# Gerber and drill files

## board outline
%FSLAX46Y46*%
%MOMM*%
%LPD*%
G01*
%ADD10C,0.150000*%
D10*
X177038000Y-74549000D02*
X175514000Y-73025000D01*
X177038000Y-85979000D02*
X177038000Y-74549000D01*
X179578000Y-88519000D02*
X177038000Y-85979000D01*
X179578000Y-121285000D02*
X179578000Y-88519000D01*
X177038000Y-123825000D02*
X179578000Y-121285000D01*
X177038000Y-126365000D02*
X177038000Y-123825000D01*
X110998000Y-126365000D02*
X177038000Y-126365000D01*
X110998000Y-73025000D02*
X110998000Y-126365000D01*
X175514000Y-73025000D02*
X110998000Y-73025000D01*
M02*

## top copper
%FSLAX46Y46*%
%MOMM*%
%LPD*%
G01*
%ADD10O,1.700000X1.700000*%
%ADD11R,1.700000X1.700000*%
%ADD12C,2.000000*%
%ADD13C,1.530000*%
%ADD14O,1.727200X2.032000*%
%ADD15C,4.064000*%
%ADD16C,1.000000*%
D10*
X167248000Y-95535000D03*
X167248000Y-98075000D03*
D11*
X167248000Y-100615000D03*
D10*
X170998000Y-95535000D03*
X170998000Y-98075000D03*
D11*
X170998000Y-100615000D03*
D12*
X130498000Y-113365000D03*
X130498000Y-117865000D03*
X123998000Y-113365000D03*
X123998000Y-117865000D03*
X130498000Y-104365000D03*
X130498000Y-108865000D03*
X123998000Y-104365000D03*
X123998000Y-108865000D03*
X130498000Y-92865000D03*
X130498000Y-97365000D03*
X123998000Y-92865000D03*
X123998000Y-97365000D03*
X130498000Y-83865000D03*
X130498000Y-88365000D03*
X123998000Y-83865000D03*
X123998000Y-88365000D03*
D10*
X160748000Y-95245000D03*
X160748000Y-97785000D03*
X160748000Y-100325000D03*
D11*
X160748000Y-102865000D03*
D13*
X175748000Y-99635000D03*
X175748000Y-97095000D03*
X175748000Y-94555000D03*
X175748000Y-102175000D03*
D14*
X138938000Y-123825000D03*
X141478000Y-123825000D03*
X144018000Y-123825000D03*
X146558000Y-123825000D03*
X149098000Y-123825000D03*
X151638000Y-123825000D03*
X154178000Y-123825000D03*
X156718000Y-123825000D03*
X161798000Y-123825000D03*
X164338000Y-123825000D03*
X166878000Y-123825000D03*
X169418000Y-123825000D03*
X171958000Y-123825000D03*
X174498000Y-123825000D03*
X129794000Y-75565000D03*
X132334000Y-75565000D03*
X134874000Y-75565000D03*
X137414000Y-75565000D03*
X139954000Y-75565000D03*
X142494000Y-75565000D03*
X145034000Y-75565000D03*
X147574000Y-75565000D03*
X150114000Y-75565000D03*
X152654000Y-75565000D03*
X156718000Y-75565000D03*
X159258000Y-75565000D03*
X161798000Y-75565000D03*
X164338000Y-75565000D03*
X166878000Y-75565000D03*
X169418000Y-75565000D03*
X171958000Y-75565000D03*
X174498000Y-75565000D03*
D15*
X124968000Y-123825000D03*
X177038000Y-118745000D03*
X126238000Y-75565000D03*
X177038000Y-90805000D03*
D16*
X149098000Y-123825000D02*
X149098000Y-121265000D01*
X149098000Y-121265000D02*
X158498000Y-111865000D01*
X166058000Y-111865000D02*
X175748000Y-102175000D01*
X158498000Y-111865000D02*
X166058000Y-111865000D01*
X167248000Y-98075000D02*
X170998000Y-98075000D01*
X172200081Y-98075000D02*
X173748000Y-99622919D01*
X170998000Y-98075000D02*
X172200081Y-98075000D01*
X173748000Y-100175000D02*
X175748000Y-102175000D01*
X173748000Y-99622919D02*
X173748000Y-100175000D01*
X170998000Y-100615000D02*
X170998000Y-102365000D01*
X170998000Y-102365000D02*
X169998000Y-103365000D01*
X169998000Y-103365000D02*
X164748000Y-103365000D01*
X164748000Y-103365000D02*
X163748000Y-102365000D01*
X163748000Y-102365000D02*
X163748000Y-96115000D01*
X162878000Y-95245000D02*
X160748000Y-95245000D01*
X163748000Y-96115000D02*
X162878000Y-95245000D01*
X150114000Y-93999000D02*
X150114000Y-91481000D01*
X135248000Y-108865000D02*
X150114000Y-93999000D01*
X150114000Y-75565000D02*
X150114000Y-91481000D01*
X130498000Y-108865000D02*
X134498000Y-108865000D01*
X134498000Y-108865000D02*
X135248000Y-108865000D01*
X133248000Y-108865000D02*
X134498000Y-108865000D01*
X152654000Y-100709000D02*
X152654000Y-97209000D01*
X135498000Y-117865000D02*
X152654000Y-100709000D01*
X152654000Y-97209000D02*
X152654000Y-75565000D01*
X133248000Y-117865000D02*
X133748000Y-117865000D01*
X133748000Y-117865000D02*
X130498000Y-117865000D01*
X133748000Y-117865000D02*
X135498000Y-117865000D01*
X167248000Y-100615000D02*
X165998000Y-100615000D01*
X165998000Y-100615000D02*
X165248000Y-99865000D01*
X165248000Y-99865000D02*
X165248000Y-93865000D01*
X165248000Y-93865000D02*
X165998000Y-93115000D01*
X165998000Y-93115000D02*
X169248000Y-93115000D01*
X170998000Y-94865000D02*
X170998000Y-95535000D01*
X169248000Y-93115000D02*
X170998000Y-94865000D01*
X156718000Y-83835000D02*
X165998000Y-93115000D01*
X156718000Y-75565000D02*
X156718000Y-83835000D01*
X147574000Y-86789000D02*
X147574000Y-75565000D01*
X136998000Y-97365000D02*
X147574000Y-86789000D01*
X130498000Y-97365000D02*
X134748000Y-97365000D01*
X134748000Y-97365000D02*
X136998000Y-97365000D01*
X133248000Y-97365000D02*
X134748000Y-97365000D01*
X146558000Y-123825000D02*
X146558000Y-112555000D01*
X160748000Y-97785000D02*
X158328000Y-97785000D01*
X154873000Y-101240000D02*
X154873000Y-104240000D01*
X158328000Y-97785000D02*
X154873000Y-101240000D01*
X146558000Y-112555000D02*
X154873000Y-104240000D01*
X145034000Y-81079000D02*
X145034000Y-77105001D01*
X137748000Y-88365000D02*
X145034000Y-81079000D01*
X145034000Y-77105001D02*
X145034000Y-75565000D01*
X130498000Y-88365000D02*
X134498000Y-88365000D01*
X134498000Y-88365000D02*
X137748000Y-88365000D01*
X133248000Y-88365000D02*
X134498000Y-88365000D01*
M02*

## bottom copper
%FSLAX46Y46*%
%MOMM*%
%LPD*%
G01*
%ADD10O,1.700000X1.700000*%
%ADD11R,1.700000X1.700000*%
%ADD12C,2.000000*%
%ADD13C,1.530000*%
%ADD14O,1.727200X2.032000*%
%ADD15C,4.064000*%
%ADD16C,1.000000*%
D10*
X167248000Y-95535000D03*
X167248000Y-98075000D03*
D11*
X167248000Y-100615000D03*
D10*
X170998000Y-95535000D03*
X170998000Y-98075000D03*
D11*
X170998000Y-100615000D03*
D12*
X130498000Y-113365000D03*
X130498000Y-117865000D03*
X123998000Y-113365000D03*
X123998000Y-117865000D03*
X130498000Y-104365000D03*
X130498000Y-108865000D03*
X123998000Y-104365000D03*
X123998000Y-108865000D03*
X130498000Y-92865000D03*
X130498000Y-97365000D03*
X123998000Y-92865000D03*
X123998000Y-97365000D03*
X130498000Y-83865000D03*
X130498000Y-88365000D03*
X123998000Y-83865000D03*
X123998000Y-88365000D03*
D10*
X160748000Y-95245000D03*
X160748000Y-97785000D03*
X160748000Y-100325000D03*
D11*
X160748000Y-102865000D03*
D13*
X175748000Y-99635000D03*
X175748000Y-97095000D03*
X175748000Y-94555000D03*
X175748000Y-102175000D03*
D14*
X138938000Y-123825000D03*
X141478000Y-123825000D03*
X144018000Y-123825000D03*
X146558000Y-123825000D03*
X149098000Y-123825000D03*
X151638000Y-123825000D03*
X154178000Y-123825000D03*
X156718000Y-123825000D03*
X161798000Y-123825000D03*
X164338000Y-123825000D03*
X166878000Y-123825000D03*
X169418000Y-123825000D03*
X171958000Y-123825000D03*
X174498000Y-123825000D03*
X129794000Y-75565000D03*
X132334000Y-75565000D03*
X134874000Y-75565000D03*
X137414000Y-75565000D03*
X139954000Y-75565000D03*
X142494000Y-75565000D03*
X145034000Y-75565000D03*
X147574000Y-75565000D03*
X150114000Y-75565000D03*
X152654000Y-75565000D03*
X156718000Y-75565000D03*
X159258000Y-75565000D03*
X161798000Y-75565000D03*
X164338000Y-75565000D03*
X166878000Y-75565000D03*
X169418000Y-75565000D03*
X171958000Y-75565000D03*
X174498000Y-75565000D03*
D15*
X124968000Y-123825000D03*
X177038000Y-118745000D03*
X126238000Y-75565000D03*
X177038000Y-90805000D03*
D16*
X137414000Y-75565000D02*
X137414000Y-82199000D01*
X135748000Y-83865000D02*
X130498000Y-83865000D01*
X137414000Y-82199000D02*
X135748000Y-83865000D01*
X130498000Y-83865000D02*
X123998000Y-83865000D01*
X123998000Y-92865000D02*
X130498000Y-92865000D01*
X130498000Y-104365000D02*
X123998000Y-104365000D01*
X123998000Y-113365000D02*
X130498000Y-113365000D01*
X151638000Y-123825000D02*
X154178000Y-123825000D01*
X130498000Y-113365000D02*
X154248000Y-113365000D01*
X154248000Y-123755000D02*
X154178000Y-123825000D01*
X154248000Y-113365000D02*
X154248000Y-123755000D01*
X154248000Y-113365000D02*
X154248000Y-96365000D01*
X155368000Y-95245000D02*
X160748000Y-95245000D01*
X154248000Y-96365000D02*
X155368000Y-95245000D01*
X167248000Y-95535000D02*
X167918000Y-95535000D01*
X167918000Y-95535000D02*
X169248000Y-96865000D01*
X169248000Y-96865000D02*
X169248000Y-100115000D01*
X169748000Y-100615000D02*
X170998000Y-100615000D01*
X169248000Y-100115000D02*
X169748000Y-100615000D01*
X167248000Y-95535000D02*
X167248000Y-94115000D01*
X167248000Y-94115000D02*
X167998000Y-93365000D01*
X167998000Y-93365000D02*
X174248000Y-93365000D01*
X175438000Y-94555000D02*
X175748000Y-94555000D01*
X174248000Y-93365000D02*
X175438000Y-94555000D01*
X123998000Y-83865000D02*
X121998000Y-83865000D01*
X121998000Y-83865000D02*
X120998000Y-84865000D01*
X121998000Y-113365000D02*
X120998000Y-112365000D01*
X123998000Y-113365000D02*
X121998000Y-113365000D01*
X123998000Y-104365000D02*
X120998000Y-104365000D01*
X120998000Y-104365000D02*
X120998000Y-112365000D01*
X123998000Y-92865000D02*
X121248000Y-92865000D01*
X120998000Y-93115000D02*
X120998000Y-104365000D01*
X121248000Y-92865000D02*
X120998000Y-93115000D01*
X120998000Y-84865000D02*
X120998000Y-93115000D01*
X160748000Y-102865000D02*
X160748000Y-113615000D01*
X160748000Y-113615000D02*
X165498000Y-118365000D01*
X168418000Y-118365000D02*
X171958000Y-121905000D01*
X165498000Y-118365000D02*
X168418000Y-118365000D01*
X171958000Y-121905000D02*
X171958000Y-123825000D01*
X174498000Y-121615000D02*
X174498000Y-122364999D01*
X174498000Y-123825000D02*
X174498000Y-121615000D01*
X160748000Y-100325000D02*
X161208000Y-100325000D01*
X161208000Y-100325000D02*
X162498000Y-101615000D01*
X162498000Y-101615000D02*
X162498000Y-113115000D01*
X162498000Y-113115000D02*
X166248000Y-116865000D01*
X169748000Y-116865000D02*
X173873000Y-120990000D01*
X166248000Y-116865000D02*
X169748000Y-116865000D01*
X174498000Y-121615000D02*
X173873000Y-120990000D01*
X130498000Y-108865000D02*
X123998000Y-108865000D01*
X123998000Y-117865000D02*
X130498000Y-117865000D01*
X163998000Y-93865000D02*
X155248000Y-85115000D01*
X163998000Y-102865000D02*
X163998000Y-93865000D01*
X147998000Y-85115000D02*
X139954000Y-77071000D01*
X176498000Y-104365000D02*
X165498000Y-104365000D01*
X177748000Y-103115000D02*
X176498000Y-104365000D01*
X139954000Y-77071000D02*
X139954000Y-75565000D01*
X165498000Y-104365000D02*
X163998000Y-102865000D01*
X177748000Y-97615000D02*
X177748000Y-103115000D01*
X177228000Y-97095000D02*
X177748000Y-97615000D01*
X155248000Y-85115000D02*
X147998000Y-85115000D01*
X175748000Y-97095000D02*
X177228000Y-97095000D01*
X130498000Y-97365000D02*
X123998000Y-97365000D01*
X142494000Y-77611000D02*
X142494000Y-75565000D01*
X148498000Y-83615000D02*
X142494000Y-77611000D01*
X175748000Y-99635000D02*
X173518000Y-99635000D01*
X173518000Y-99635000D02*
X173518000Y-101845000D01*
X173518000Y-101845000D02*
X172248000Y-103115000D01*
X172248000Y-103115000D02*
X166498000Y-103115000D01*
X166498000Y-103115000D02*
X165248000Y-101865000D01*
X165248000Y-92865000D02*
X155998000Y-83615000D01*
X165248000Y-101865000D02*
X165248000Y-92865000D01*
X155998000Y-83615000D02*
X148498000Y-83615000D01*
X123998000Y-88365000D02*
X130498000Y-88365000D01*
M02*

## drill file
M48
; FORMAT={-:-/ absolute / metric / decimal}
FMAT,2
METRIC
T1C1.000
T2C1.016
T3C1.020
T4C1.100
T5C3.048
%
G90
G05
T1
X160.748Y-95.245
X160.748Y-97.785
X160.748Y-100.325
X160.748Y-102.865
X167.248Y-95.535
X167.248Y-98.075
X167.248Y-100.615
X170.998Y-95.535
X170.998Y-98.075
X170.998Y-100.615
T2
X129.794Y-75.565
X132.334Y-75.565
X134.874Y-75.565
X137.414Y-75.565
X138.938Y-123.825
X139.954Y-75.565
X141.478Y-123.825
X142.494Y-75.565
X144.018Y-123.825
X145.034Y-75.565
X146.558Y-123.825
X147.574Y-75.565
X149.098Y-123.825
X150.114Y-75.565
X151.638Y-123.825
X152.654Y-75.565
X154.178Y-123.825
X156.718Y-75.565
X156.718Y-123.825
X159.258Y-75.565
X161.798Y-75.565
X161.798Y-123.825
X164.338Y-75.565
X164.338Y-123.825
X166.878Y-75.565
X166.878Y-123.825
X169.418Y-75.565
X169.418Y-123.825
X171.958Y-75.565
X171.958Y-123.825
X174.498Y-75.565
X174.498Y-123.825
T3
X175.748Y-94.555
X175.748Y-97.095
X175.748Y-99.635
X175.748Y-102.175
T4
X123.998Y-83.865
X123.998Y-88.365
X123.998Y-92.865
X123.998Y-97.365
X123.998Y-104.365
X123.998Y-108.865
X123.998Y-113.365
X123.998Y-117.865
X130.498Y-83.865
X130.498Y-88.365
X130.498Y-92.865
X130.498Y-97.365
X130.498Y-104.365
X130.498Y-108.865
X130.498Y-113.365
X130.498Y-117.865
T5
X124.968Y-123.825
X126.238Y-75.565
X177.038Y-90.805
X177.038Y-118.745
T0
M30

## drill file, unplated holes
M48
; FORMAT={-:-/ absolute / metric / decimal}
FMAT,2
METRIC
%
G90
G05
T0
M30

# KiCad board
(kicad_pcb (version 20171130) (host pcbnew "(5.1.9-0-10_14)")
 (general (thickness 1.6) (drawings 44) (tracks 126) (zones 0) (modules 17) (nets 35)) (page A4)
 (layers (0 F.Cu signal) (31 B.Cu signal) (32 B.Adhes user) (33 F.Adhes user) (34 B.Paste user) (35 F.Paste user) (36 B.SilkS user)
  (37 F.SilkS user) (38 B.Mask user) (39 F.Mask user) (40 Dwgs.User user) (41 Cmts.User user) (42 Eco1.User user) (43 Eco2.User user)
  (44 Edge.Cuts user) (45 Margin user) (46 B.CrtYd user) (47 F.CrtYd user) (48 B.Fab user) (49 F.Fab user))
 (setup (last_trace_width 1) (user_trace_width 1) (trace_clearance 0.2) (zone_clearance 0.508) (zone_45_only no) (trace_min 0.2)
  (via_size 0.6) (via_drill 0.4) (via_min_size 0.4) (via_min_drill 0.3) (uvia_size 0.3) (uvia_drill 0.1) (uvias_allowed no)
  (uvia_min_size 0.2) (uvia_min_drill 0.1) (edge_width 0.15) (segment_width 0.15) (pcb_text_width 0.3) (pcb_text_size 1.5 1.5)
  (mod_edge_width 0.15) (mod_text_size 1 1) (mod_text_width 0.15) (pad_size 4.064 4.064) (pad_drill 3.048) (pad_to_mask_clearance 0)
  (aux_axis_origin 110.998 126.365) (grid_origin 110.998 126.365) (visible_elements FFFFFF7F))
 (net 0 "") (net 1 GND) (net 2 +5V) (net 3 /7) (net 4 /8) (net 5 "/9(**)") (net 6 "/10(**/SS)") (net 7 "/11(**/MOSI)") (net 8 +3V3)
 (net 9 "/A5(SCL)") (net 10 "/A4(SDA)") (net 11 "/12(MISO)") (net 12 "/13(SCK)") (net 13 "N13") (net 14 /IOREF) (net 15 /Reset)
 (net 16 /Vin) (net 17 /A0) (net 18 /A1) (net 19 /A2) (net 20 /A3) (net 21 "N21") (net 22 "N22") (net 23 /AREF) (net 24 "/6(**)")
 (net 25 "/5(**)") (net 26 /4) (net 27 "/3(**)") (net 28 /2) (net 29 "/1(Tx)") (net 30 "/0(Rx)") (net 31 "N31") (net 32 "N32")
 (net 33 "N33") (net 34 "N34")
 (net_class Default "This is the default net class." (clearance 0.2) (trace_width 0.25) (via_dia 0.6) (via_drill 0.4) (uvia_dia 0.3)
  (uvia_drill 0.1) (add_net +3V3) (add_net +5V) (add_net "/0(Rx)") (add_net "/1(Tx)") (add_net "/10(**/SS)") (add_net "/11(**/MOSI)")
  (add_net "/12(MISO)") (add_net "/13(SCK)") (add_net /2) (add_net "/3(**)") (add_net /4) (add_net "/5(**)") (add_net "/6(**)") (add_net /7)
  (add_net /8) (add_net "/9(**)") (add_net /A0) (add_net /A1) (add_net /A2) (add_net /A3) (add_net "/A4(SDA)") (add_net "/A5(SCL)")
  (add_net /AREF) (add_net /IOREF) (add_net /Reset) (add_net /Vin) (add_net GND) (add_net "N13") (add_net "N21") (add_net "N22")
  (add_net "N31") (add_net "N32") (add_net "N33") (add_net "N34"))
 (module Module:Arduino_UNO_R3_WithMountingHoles (layer B.Cu) (at 138.998 123.765)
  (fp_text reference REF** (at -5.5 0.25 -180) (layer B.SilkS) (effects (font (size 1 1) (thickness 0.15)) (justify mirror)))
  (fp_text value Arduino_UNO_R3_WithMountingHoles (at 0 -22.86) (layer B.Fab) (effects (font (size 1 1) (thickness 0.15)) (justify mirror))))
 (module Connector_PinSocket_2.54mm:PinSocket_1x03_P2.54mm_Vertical (layer F.Cu) (at 167.248 100.615 180)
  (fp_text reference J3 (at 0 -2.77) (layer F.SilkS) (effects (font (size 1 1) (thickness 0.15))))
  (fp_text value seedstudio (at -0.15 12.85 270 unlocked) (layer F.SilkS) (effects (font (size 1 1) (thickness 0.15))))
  (pad 3 thru_hole oval (at 0 5.08 180) (size 1.7 1.7) (drill 1) (layers *.Cu *.Mask) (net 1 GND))
  (pad 2 thru_hole oval (at 0 2.54 180) (size 1.7 1.7) (drill 1) (layers *.Cu *.Mask) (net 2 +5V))
  (pad 1 thru_hole rect (at 0 0 180) (size 1.7 1.7) (drill 1) (layers *.Cu *.Mask) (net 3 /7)))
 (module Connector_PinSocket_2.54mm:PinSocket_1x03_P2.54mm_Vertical (layer F.Cu) (at 170.998 100.615 180)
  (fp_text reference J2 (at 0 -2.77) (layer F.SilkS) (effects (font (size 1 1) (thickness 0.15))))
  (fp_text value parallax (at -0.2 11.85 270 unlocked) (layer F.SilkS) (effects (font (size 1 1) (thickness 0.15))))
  (pad 3 thru_hole oval (at 0 5.08 180) (size 1.7 1.7) (drill 1) (layers *.Cu *.Mask) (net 3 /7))
  (pad 2 thru_hole oval (at 0 2.54 180) (size 1.7 1.7) (drill 1) (layers *.Cu *.Mask) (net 2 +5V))
  (pad 1 thru_hole rect (at 0 0 180) (size 1.7 1.7) (drill 1) (layers *.Cu *.Mask) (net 1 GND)))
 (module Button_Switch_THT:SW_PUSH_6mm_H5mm (layer F.Cu) (at 123.998 113.365)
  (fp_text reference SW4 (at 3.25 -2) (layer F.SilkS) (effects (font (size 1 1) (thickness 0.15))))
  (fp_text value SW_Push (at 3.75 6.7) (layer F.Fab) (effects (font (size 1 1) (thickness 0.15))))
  (pad 1 thru_hole circle (at 6.5 0 90) (size 2 2) (drill 1.1) (layers *.Cu *.Mask) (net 1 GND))
  (pad 2 thru_hole circle (at 6.5 4.5 90) (size 2 2) (drill 1.1) (layers *.Cu *.Mask) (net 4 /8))
  (pad 1 thru_hole circle (at 0 0 90) (size 2 2) (drill 1.1) (layers *.Cu *.Mask) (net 1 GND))
  (pad 2 thru_hole circle (at 0 4.5 90) (size 2 2) (drill 1.1) (layers *.Cu *.Mask) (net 4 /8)))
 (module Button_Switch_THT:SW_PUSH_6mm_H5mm (layer F.Cu) (at 123.998 104.365)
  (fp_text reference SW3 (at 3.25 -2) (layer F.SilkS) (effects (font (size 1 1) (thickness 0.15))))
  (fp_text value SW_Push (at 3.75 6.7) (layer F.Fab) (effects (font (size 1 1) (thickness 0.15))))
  (pad 1 thru_hole circle (at 6.5 0 90) (size 2 2) (drill 1.1) (layers *.Cu *.Mask) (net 1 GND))
  (pad 2 thru_hole circle (at 6.5 4.5 90) (size 2 2) (drill 1.1) (layers *.Cu *.Mask) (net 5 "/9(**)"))
  (pad 1 thru_hole circle (at 0 0 90) (size 2 2) (drill 1.1) (layers *.Cu *.Mask) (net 1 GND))
  (pad 2 thru_hole circle (at 0 4.5 90) (size 2 2) (drill 1.1) (layers *.Cu *.Mask) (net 5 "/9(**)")))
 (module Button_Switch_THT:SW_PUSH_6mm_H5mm (layer F.Cu) (at 123.998 92.865)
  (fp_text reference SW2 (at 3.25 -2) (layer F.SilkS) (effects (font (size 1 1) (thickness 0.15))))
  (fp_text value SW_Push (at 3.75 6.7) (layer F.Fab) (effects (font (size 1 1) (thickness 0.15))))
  (pad 1 thru_hole circle (at 6.5 0 90) (size 2 2) (drill 1.1) (layers *.Cu *.Mask) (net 1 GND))
  (pad 2 thru_hole circle (at 6.5 4.5 90) (size 2 2) (drill 1.1) (layers *.Cu *.Mask) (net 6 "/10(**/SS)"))
  (pad 1 thru_hole circle (at 0 0 90) (size 2 2) (drill 1.1) (layers *.Cu *.Mask) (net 1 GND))
  (pad 2 thru_hole circle (at 0 4.5 90) (size 2 2) (drill 1.1) (layers *.Cu *.Mask) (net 6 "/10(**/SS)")))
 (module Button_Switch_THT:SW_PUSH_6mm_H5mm (layer F.Cu) (at 123.998 83.865)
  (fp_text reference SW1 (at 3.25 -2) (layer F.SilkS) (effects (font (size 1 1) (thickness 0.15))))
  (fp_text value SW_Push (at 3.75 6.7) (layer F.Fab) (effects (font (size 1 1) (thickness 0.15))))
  (pad 1 thru_hole circle (at 6.5 0 90) (size 2 2) (drill 1.1) (layers *.Cu *.Mask) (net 1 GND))
  (pad 2 thru_hole circle (at 6.5 4.5 90) (size 2 2) (drill 1.1) (layers *.Cu *.Mask) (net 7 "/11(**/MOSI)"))
  (pad 1 thru_hole circle (at 0 0 90) (size 2 2) (drill 1.1) (layers *.Cu *.Mask) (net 1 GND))
  (pad 2 thru_hole circle (at 0 4.5 90) (size 2 2) (drill 1.1) (layers *.Cu *.Mask) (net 7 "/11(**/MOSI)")))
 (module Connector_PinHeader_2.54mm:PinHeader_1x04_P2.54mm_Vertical (layer F.Cu) (at 160.748 102.865 180)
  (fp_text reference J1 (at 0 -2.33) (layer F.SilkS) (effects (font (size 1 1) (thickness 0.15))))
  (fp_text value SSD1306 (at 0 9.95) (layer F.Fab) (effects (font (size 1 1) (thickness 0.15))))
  (pad 4 thru_hole oval (at 0 7.62 180) (size 1.7 1.7) (drill 1) (layers *.Cu *.Mask) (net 1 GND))
  (pad 3 thru_hole oval (at 0 5.08 180) (size 1.7 1.7) (drill 1) (layers *.Cu *.Mask) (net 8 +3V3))
  (pad 2 thru_hole oval (at 0 2.54 180) (size 1.7 1.7) (drill 1) (layers *.Cu *.Mask) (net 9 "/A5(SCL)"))
  (pad 1 thru_hole rect (at 0 0 180) (size 1.7 1.7) (drill 1) (layers *.Cu *.Mask) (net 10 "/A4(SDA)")))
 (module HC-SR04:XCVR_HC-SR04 (layer F.Cu) (at 175.748 98.365 90)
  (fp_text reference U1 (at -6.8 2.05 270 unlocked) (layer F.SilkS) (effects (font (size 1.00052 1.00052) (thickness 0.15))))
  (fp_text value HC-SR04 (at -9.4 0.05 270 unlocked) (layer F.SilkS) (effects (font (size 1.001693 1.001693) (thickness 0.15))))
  (pad 2 thru_hole circle (at -1.27 0 90) (size 1.53 1.53) (drill 1.02) (layers *.Cu *.Mask) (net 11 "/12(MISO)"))
  (pad 3 thru_hole circle (at 1.27 0 90) (size 1.53 1.53) (drill 1.02) (layers *.Cu *.Mask) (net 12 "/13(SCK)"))
  (pad 4 thru_hole circle (at 3.81 0 90) (size 1.53 1.53) (drill 1.02) (layers *.Cu *.Mask) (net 1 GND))
  (pad 1 thru_hole circle (at -3.81 0 90) (size 1.53 1.53) (drill 1.02) (layers *.Cu *.Mask) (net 2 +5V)))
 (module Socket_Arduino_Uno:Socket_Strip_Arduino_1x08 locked (layer F.Cu) (at 138.938 123.825)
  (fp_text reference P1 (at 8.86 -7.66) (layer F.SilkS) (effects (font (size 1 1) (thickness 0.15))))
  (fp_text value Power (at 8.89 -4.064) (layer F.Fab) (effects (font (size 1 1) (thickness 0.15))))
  (pad 1 thru_hole oval (at 0 0) (size 1.7272 2.032) (drill 1.016) (layers *.Cu *.Mask F.SilkS) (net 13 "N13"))
  (pad 2 thru_hole oval (at 2.54 0) (size 1.7272 2.032) (drill 1.016) (layers *.Cu *.Mask F.SilkS) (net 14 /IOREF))
  (pad 3 thru_hole oval (at 5.08 0) (size 1.7272 2.032) (drill 1.016) (layers *.Cu *.Mask F.SilkS) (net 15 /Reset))
  (pad 4 thru_hole oval (at 7.62 0) (size 1.7272 2.032) (drill 1.016) (layers *.Cu *.Mask F.SilkS) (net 8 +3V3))
  (pad 5 thru_hole oval (at 10.16 0) (size 1.7272 2.032) (drill 1.016) (layers *.Cu *.Mask F.SilkS) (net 2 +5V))
  (pad 6 thru_hole oval (at 12.7 0) (size 1.7272 2.032) (drill 1.016) (layers *.Cu *.Mask F.SilkS) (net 1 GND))
  (pad 7 thru_hole oval (at 15.24 0) (size 1.7272 2.032) (drill 1.016) (layers *.Cu *.Mask F.SilkS) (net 1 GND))
  (pad 8 thru_hole oval (at 17.78 0) (size 1.7272 2.032) (drill 1.016) (layers *.Cu *.Mask F.SilkS) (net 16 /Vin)))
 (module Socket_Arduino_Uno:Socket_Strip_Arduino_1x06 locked (layer F.Cu) (at 161.798 123.825)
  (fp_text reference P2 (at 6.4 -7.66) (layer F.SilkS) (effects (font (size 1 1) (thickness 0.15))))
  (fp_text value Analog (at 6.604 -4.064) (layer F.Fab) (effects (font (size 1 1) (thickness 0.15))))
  (pad 1 thru_hole oval (at 0 0) (size 1.7272 2.032) (drill 1.016) (layers *.Cu *.Mask F.SilkS) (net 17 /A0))
  (pad 2 thru_hole oval (at 2.54 0) (size 1.7272 2.032) (drill 1.016) (layers *.Cu *.Mask F.SilkS) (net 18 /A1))
  (pad 3 thru_hole oval (at 5.08 0) (size 1.7272 2.032) (drill 1.016) (layers *.Cu *.Mask F.SilkS) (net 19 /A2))
  (pad 4 thru_hole oval (at 7.62 0) (size 1.7272 2.032) (drill 1.016) (layers *.Cu *.Mask F.SilkS) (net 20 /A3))
  (pad 5 thru_hole oval (at 10.16 0) (size 1.7272 2.032) (drill 1.016) (layers *.Cu *.Mask F.SilkS) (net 10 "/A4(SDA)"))
  (pad 6 thru_hole oval (at 12.7 0) (size 1.7272 2.032) (drill 1.016) (layers *.Cu *.Mask F.SilkS) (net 9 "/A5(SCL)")))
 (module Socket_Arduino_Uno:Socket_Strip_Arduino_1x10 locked (layer F.Cu) (at 129.794 75.565)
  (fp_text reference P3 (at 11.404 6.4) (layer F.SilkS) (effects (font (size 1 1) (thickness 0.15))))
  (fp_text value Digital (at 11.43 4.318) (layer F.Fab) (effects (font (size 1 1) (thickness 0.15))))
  (pad 1 thru_hole oval (at 0 0) (size 1.7272 2.032) (drill 1.016) (layers *.Cu *.Mask F.SilkS) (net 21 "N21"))
  (pad 2 thru_hole oval (at 2.54 0) (size 1.7272 2.032) (drill 1.016) (layers *.Cu *.Mask F.SilkS) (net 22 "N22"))
  (pad 3 thru_hole oval (at 5.08 0) (size 1.7272 2.032) (drill 1.016) (layers *.Cu *.Mask F.SilkS) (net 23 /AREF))
  (pad 4 thru_hole oval (at 7.62 0) (size 1.7272 2.032) (drill 1.016) (layers *.Cu *.Mask F.SilkS) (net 1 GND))
  (pad 5 thru_hole oval (at 10.16 0) (size 1.7272 2.032) (drill 1.016) (layers *.Cu *.Mask F.SilkS) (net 12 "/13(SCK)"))
  (pad 6 thru_hole oval (at 12.7 0) (size 1.7272 2.032) (drill 1.016) (layers *.Cu *.Mask F.SilkS) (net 11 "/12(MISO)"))
  (pad 7 thru_hole oval (at 15.24 0) (size 1.7272 2.032) (drill 1.016) (layers *.Cu *.Mask F.SilkS) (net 7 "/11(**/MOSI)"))
  (pad 8 thru_hole oval (at 17.78 0) (size 1.7272 2.032) (drill 1.016) (layers *.Cu *.Mask F.SilkS) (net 6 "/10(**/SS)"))
  (pad 9 thru_hole oval (at 20.32 0) (size 1.7272 2.032) (drill 1.016) (layers *.Cu *.Mask F.SilkS) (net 5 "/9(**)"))
  (pad 10 thru_hole oval (at 22.86 0) (size 1.7272 2.032) (drill 1.016) (layers *.Cu *.Mask F.SilkS) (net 4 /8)))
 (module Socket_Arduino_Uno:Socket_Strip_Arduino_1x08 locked (layer F.Cu) (at 156.718 75.565)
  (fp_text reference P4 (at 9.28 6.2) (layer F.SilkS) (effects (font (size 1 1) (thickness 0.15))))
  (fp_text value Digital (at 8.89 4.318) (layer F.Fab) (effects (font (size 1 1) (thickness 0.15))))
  (pad 1 thru_hole oval (at 0 0) (size 1.7272 2.032) (drill 1.016) (layers *.Cu *.Mask F.SilkS) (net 3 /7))
  (pad 2 thru_hole oval (at 2.54 0) (size 1.7272 2.032) (drill 1.016) (layers *.Cu *.Mask F.SilkS) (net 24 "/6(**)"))
  (pad 3 thru_hole oval (at 5.08 0) (size 1.7272 2.032) (drill 1.016) (layers *.Cu *.Mask F.SilkS) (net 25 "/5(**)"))
  (pad 4 thru_hole oval (at 7.62 0) (size 1.7272 2.032) (drill 1.016) (layers *.Cu *.Mask F.SilkS) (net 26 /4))
  (pad 5 thru_hole oval (at 10.16 0) (size 1.7272 2.032) (drill 1.016) (layers *.Cu *.Mask F.SilkS) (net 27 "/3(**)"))
  (pad 6 thru_hole oval (at 12.7 0) (size 1.7272 2.032) (drill 1.016) (layers *.Cu *.Mask F.SilkS) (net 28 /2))
  (pad 7 thru_hole oval (at 15.24 0) (size 1.7272 2.032) (drill 1.016) (layers *.Cu *.Mask F.SilkS) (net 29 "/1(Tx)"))
  (pad 8 thru_hole oval (at 17.78 0) (size 1.7272 2.032) (drill 1.016) (layers *.Cu *.Mask F.SilkS) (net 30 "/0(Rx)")))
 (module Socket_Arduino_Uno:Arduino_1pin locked (layer F.Cu) (at 124.968 123.825)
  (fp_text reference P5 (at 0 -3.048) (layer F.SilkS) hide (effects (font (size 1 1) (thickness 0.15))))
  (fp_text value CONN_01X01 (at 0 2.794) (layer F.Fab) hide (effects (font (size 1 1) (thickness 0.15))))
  (pad 1 thru_hole circle (at 0 0) (size 4.064 4.064) (drill 3.048) (layers *.Cu *.Mask F.SilkS) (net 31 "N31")))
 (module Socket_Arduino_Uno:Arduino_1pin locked (layer F.Cu) (at 177.038 118.745)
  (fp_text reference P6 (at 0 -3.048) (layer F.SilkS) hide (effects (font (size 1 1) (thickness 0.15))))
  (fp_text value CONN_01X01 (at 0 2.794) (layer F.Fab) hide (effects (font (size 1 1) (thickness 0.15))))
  (pad 1 thru_hole circle (at 0 0) (size 4.064 4.064) (drill 3.048) (layers *.Cu *.Mask F.SilkS) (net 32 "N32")))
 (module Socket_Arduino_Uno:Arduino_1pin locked (layer F.Cu) (at 126.238 75.565)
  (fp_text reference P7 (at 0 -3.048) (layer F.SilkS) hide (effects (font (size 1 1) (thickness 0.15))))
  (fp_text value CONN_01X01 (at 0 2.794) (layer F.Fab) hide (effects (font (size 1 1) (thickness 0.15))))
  (pad 1 thru_hole circle (at 0 0) (size 4.064 4.064) (drill 3.048) (layers *.Cu *.Mask F.SilkS) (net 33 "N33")))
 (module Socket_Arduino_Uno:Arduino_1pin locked (layer F.Cu) (at 177.038 90.805)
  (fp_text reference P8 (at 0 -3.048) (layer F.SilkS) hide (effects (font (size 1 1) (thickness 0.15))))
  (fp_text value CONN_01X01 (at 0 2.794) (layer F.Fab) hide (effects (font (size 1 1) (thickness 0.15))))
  (pad 1 thru_hole circle (at 0 0) (size 4.064 4.064) (drill 3.048) (layers *.Cu *.Mask F.SilkS) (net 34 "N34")))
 (gr_line (start 177.038 74.549) (end 175.514 73.025) (angle 90) (layer Edge.Cuts) (width 0.15))
 (gr_line (start 177.038 85.979) (end 177.038 74.549) (angle 90) (layer Edge.Cuts) (width 0.15))
 (gr_line (start 179.578 88.519) (end 177.038 85.979) (angle 90) (layer Edge.Cuts) (width 0.15))
 (gr_line (start 179.578 121.285) (end 179.578 88.519) (angle 90) (layer Edge.Cuts) (width 0.15))
 (gr_line (start 177.038 123.825) (end 179.578 121.285) (angle 90) (layer Edge.Cuts) (width 0.15))
 (gr_line (start 177.038 126.365) (end 177.038 123.825) (angle 90) (layer Edge.Cuts) (width 0.15))
 (gr_line (start 110.998 126.365) (end 177.038 126.365) (angle 90) (layer Edge.Cuts) (width 0.15))
 (gr_line (start 110.998 73.025) (end 110.998 126.365) (angle 90) (layer Edge.Cuts) (width 0.15))
 (gr_line (start 175.514 73.025) (end 110.998 73.025) (angle 90) (layer Edge.Cuts) (width 0.15))
 (segment (start 149.098 123.825) (end 149.098 121.265) (width 1) (layer F.Cu) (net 2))
 (segment (start 149.098 121.265) (end 158.498 111.865) (width 1) (layer F.Cu) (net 2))
 (segment (start 166.058 111.865) (end 175.748 102.175) (width 1) (layer F.Cu) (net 2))
 (segment (start 158.498 111.865) (end 166.058 111.865) (width 1) (layer F.Cu) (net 2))
 (segment (start 167.248 98.075) (end 170.998 98.075) (width 1) (layer F.Cu) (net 2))
 (segment (start 172.200081 98.075) (end 173.748 99.622919) (width 1) (layer F.Cu) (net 2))
 (segment (start 170.998 98.075) (end 172.200081 98.075) (width 1) (layer F.Cu) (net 2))
 (segment (start 173.748 100.175) (end 175.748 102.175) (width 1) (layer F.Cu) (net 2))
 (segment (start 173.748 99.622919) (end 173.748 100.175) (width 1) (layer F.Cu) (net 2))
 (segment (start 170.998 100.615) (end 170.998 102.365) (width 1) (layer F.Cu) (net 1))
 (segment (start 170.998 102.365) (end 169.998 103.365) (width 1) (layer F.Cu) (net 1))
 (segment (start 169.998 103.365) (end 164.748 103.365) (width 1) (layer F.Cu) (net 1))
 (segment (start 164.748 103.365) (end 163.748 102.365) (width 1) (layer F.Cu) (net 1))
 (segment (start 163.748 102.365) (end 163.748 96.115) (width 1) (layer F.Cu) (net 1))
 (segment (start 162.878 95.245) (end 160.748 95.245) (width 1) (layer F.Cu) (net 1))
 (segment (start 163.748 96.115) (end 162.878 95.245) (width 1) (layer F.Cu) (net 1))
 (segment (start 137.414 75.565) (end 137.414 82.199) (width 1) (layer B.Cu) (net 1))
 (segment (start 135.748 83.865) (end 130.498 83.865) (width 1) (layer B.Cu) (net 1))
 (segment (start 137.414 82.199) (end 135.748 83.865) (width 1) (layer B.Cu) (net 1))
 (segment (start 130.498 83.865) (end 123.998 83.865) (width 1) (layer B.Cu) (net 1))
 (segment (start 123.998 92.865) (end 130.498 92.865) (width 1) (layer B.Cu) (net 1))
 (segment (start 130.498 104.365) (end 123.998 104.365) (width 1) (layer B.Cu) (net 1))
 (segment (start 123.998 113.365) (end 130.498 113.365) (width 1) (layer B.Cu) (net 1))
 (segment (start 151.638 123.825) (end 154.178 123.825) (width 1) (layer B.Cu) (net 1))
 (segment (start 130.498 113.365) (end 154.248 113.365) (width 1) (layer B.Cu) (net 1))
 (segment (start 154.248 123.755) (end 154.178 123.825) (width 1) (layer B.Cu) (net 1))
 (segment (start 154.248 113.365) (end 154.248 123.755) (width 1) (layer B.Cu) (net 1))
 (segment (start 154.248 113.365) (end 154.248 96.365) (width 1) (layer B.Cu) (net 1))
 (segment (start 155.368 95.245) (end 160.748 95.245) (width 1) (layer B.Cu) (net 1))
 (segment (start 154.248 96.365) (end 155.368 95.245) (width 1) (layer B.Cu) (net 1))
 (segment (start 167.248 95.535) (end 167.918 95.535) (width 1) (layer B.Cu) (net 1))
 (segment (start 167.918 95.535) (end 169.248 96.865) (width 1) (layer B.Cu) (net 1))
 (segment (start 169.248 96.865) (end 169.248 100.115) (width 1) (layer B.Cu) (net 1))
 (segment (start 169.748 100.615) (end 170.998 100.615) (width 1) (layer B.Cu) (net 1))
 (segment (start 169.248 100.115) (end 169.748 100.615) (width 1) (layer B.Cu) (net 1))
 (segment (start 167.248 95.535) (end 167.248 94.115) (width 1) (layer B.Cu) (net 1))
 (segment (start 167.248 94.115) (end 167.998 93.365) (width 1) (layer B.Cu) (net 1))
 (segment (start 167.998 93.365) (end 174.248 93.365) (width 1) (layer B.Cu) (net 1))
 (segment (start 175.438 94.555) (end 175.748 94.555) (width 1) (layer B.Cu) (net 1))
 (segment (start 174.248 93.365) (end 175.438 94.555) (width 1) (layer B.Cu) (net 1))
 (segment (start 123.998 83.865) (end 121.998 83.865) (width 1) (layer B.Cu) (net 1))
 (segment (start 121.998 83.865) (end 120.998 84.865) (width 1) (layer B.Cu) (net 1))
 (segment (start 121.998 113.365) (end 120.998 112.365) (width 1) (layer B.Cu) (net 1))
 (segment (start 123.998 113.365) (end 121.998 113.365) (width 1) (layer B.Cu) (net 1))
 (segment (start 123.998 104.365) (end 120.998 104.365) (width 1) (layer B.Cu) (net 1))
 (segment (start 120.998 104.365) (end 120.998 112.365) (width 1) (layer B.Cu) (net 1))
 (segment (start 123.998 92.865) (end 121.248 92.865) (width 1) (layer B.Cu) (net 1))
 (segment (start 120.998 93.115) (end 120.998 104.365) (width 1) (layer B.Cu) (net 1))
 (segment (start 121.248 92.865) (end 120.998 93.115) (width 1) (layer B.Cu) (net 1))
 (segment (start 120.998 84.865) (end 120.998 93.115) (width 1) (layer B.Cu) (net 1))
 (segment (start 160.748 102.865) (end 160.748 113.615) (width 1) (layer B.Cu) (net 10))
 (segment (start 160.748 113.615) (end 165.498 118.365) (width 1) (layer B.Cu) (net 10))
 (segment (start 168.418 118.365) (end 171.958 121.905) (width 1) (layer B.Cu) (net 10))
 (segment (start 165.498 118.365) (end 168.418 118.365) (width 1) (layer B.Cu) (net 10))
 (segment (start 171.958 121.905) (end 171.958 123.825) (width 1) (layer B.Cu) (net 10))
 (segment (start 174.498 121.615) (end 174.498 122.364999) (width 1) (layer B.Cu) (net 9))
 (segment (start 174.498 123.825) (end 174.498 121.615) (width 1) (layer B.Cu) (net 9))
 (segment (start 160.748 100.325) (end 161.208 100.325) (width 1) (layer B.Cu) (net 9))
 (segment (start 161.208 100.325) (end 162.498 101.615) (width 1) (layer B.Cu) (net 9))
 (segment (start 162.498 101.615) (end 162.498 113.115) (width 1) (layer B.Cu) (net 9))
 (segment (start 162.498 113.115) (end 166.248 116.865) (width 1) (layer B.Cu) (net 9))
 (segment (start 169.748 116.865) (end 173.873 120.99) (width 1) (layer B.Cu) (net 9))
 (segment (start 166.248 116.865) (end 169.748 116.865) (width 1) (layer B.Cu) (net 9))
 (segment (start 174.498 121.615) (end 173.873 120.99) (width 1) (layer B.Cu) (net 9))
 (segment (start 150.114 93.999) (end 150.114 91.481) (width 1) (layer F.Cu) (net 5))
 (segment (start 135.248 108.865) (end 150.114 93.999) (width 1) (layer F.Cu) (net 5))
 (segment (start 150.114 75.565) (end 150.114 91.481) (width 1) (layer F.Cu) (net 5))
 (segment (start 130.498 108.865) (end 123.998 108.865) (width 1) (layer B.Cu) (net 5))
 (segment (start 130.498 108.865) (end 134.498 108.865) (width 1) (layer F.Cu) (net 5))
 (segment (start 134.498 108.865) (end 135.248 108.865) (width 1) (layer F.Cu) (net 5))
 (segment (start 133.248 108.865) (end 134.498 108.865) (width 1) (layer F.Cu) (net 5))
 (segment (start 152.654 100.709) (end 152.654 97.209) (width 1) (layer F.Cu) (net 4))
 (segment (start 135.498 117.865) (end 152.654 100.709) (width 1) (layer F.Cu) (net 4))
 (segment (start 152.654 97.209) (end 152.654 75.565) (width 1) (layer F.Cu) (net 4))
 (segment (start 123.998 117.865) (end 130.498 117.865) (width 1) (layer B.Cu) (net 4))
 (segment (start 133.248 117.865) (end 133.748 117.865) (width 1) (layer F.Cu) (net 4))
 (segment (start 133.748 117.865) (end 130.498 117.865) (width 1) (layer F.Cu) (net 4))
 (segment (start 133.748 117.865) (end 135.498 117.865) (width 1) (layer F.Cu) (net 4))
 (segment (start 167.248 100.615) (end 165.998 100.615) (width 1) (layer F.Cu) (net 3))
 (segment (start 165.998 100.615) (end 165.248 99.865) (width 1) (layer F.Cu) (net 3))
 (segment (start 165.248 99.865) (end 165.248 93.865) (width 1) (layer F.Cu) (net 3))
 (segment (start 165.248 93.865) (end 165.998 93.115) (width 1) (layer F.Cu) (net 3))
 (segment (start 165.998 93.115) (end 169.248 93.115) (width 1) (layer F.Cu) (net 3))
 (segment (start 170.998 94.865) (end 170.998 95.535) (width 1) (layer F.Cu) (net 3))
 (segment (start 169.248 93.115) (end 170.998 94.865) (width 1) (layer F.Cu) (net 3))
 (segment (start 156.718 83.835) (end 165.998 93.115) (width 1) (layer F.Cu) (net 3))
 (segment (start 156.718 75.565) (end 156.718 83.835) (width 1) (layer F.Cu) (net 3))
 (segment (start 163.998 93.865) (end 155.248 85.115) (width 1) (layer B.Cu) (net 12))
 (segment (start 163.998 102.865) (end 163.998 93.865) (width 1) (layer B.Cu) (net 12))
 (segment (start 147.998 85.115) (end 139.954 77.071) (width 1) (layer B.Cu) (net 12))
 (segment (start 176.498 104.365) (end 165.498 104.365) (width 1) (layer B.Cu) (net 12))
 (segment (start 177.748 103.115) (end 176.498 104.365) (width 1) (layer B.Cu) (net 12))
 (segment (start 139.954 77.071) (end 139.954 75.565) (width 1) (layer B.Cu) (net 12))
 (segment (start 165.498 104.365) (end 163.998 102.865) (width 1) (layer B.Cu) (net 12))
 (segment (start 177.748 97.615) (end 177.748 103.115) (width 1) (layer B.Cu) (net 12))
 (segment (start 177.228 97.095) (end 177.748 97.615) (width 1) (layer B.Cu) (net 12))
 (segment (start 155.248 85.115) (end 147.998 85.115) (width 1) (layer B.Cu) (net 12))
 (segment (start 175.748 97.095) (end 177.228 97.095) (width 1) (layer B.Cu) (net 12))
 (segment (start 147.574 86.789) (end 147.574 75.565) (width 1) (layer F.Cu) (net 6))
 (segment (start 136.998 97.365) (end 147.574 86.789) (width 1) (layer F.Cu) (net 6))
 (segment (start 130.498 97.365) (end 123.998 97.365) (width 1) (layer B.Cu) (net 6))
 (segment (start 130.498 97.365) (end 134.748 97.365) (width 1) (layer F.Cu) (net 6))
 (segment (start 134.748 97.365) (end 136.998 97.365) (width 1) (layer F.Cu) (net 6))
 (segment (start 133.248 97.365) (end 134.748 97.365) (width 1) (layer F.Cu) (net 6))
 (segment (start 146.558 123.825) (end 146.558 112.555) (width 1) (layer F.Cu) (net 8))
 (segment (start 160.748 97.785) (end 158.328 97.785) (width 1) (layer F.Cu) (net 8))
 (segment (start 154.873 101.24) (end 154.873 104.24) (width 1) (layer F.Cu) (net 8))
 (segment (start 158.328 97.785) (end 154.873 101.24) (width 1) (layer F.Cu) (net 8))
 (segment (start 146.558 112.555) (end 154.873 104.24) (width 1) (layer F.Cu) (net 8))
 (segment (start 142.494 77.611) (end 142.494 75.565) (width 1) (layer B.Cu) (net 11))
 (segment (start 148.498 83.615) (end 142.494 77.611) (width 1) (layer B.Cu) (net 11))
 (segment (start 175.748 99.635) (end 173.518 99.635) (width 1) (layer B.Cu) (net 11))
 (segment (start 173.518 99.635) (end 173.518 101.845) (width 1) (layer B.Cu) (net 11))
 (segment (start 173.518 101.845) (end 172.248 103.115) (width 1) (layer B.Cu) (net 11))
 (segment (start 172.248 103.115) (end 166.498 103.115) (width 1) (layer B.Cu) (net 11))
 (segment (start 166.498 103.115) (end 165.248 101.865) (width 1) (layer B.Cu) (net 11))
 (segment (start 165.248 92.865) (end 155.998 83.615) (width 1) (layer B.Cu) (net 11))
 (segment (start 165.248 101.865) (end 165.248 92.865) (width 1) (layer B.Cu) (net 11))
 (segment (start 155.998 83.615) (end 148.498 83.615) (width 1) (layer B.Cu) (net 11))
 (segment (start 145.034 81.079) (end 145.034 77.105001) (width 1) (layer F.Cu) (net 7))
 (segment (start 137.748 88.365) (end 145.034 81.079) (width 1) (layer F.Cu) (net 7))
 (segment (start 145.034 77.105001) (end 145.034 75.565) (width 1) (layer F.Cu) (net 7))
 (segment (start 123.998 88.365) (end 130.498 88.365) (width 1) (layer B.Cu) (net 7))
 (segment (start 130.498 88.365) (end 134.498 88.365) (width 1) (layer F.Cu) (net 7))
 (segment (start 134.498 88.365) (end 137.748 88.365) (width 1) (layer F.Cu) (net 7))
 (segment (start 133.248 88.365) (end 134.498 88.365) (width 1) (layer F.Cu) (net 7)))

